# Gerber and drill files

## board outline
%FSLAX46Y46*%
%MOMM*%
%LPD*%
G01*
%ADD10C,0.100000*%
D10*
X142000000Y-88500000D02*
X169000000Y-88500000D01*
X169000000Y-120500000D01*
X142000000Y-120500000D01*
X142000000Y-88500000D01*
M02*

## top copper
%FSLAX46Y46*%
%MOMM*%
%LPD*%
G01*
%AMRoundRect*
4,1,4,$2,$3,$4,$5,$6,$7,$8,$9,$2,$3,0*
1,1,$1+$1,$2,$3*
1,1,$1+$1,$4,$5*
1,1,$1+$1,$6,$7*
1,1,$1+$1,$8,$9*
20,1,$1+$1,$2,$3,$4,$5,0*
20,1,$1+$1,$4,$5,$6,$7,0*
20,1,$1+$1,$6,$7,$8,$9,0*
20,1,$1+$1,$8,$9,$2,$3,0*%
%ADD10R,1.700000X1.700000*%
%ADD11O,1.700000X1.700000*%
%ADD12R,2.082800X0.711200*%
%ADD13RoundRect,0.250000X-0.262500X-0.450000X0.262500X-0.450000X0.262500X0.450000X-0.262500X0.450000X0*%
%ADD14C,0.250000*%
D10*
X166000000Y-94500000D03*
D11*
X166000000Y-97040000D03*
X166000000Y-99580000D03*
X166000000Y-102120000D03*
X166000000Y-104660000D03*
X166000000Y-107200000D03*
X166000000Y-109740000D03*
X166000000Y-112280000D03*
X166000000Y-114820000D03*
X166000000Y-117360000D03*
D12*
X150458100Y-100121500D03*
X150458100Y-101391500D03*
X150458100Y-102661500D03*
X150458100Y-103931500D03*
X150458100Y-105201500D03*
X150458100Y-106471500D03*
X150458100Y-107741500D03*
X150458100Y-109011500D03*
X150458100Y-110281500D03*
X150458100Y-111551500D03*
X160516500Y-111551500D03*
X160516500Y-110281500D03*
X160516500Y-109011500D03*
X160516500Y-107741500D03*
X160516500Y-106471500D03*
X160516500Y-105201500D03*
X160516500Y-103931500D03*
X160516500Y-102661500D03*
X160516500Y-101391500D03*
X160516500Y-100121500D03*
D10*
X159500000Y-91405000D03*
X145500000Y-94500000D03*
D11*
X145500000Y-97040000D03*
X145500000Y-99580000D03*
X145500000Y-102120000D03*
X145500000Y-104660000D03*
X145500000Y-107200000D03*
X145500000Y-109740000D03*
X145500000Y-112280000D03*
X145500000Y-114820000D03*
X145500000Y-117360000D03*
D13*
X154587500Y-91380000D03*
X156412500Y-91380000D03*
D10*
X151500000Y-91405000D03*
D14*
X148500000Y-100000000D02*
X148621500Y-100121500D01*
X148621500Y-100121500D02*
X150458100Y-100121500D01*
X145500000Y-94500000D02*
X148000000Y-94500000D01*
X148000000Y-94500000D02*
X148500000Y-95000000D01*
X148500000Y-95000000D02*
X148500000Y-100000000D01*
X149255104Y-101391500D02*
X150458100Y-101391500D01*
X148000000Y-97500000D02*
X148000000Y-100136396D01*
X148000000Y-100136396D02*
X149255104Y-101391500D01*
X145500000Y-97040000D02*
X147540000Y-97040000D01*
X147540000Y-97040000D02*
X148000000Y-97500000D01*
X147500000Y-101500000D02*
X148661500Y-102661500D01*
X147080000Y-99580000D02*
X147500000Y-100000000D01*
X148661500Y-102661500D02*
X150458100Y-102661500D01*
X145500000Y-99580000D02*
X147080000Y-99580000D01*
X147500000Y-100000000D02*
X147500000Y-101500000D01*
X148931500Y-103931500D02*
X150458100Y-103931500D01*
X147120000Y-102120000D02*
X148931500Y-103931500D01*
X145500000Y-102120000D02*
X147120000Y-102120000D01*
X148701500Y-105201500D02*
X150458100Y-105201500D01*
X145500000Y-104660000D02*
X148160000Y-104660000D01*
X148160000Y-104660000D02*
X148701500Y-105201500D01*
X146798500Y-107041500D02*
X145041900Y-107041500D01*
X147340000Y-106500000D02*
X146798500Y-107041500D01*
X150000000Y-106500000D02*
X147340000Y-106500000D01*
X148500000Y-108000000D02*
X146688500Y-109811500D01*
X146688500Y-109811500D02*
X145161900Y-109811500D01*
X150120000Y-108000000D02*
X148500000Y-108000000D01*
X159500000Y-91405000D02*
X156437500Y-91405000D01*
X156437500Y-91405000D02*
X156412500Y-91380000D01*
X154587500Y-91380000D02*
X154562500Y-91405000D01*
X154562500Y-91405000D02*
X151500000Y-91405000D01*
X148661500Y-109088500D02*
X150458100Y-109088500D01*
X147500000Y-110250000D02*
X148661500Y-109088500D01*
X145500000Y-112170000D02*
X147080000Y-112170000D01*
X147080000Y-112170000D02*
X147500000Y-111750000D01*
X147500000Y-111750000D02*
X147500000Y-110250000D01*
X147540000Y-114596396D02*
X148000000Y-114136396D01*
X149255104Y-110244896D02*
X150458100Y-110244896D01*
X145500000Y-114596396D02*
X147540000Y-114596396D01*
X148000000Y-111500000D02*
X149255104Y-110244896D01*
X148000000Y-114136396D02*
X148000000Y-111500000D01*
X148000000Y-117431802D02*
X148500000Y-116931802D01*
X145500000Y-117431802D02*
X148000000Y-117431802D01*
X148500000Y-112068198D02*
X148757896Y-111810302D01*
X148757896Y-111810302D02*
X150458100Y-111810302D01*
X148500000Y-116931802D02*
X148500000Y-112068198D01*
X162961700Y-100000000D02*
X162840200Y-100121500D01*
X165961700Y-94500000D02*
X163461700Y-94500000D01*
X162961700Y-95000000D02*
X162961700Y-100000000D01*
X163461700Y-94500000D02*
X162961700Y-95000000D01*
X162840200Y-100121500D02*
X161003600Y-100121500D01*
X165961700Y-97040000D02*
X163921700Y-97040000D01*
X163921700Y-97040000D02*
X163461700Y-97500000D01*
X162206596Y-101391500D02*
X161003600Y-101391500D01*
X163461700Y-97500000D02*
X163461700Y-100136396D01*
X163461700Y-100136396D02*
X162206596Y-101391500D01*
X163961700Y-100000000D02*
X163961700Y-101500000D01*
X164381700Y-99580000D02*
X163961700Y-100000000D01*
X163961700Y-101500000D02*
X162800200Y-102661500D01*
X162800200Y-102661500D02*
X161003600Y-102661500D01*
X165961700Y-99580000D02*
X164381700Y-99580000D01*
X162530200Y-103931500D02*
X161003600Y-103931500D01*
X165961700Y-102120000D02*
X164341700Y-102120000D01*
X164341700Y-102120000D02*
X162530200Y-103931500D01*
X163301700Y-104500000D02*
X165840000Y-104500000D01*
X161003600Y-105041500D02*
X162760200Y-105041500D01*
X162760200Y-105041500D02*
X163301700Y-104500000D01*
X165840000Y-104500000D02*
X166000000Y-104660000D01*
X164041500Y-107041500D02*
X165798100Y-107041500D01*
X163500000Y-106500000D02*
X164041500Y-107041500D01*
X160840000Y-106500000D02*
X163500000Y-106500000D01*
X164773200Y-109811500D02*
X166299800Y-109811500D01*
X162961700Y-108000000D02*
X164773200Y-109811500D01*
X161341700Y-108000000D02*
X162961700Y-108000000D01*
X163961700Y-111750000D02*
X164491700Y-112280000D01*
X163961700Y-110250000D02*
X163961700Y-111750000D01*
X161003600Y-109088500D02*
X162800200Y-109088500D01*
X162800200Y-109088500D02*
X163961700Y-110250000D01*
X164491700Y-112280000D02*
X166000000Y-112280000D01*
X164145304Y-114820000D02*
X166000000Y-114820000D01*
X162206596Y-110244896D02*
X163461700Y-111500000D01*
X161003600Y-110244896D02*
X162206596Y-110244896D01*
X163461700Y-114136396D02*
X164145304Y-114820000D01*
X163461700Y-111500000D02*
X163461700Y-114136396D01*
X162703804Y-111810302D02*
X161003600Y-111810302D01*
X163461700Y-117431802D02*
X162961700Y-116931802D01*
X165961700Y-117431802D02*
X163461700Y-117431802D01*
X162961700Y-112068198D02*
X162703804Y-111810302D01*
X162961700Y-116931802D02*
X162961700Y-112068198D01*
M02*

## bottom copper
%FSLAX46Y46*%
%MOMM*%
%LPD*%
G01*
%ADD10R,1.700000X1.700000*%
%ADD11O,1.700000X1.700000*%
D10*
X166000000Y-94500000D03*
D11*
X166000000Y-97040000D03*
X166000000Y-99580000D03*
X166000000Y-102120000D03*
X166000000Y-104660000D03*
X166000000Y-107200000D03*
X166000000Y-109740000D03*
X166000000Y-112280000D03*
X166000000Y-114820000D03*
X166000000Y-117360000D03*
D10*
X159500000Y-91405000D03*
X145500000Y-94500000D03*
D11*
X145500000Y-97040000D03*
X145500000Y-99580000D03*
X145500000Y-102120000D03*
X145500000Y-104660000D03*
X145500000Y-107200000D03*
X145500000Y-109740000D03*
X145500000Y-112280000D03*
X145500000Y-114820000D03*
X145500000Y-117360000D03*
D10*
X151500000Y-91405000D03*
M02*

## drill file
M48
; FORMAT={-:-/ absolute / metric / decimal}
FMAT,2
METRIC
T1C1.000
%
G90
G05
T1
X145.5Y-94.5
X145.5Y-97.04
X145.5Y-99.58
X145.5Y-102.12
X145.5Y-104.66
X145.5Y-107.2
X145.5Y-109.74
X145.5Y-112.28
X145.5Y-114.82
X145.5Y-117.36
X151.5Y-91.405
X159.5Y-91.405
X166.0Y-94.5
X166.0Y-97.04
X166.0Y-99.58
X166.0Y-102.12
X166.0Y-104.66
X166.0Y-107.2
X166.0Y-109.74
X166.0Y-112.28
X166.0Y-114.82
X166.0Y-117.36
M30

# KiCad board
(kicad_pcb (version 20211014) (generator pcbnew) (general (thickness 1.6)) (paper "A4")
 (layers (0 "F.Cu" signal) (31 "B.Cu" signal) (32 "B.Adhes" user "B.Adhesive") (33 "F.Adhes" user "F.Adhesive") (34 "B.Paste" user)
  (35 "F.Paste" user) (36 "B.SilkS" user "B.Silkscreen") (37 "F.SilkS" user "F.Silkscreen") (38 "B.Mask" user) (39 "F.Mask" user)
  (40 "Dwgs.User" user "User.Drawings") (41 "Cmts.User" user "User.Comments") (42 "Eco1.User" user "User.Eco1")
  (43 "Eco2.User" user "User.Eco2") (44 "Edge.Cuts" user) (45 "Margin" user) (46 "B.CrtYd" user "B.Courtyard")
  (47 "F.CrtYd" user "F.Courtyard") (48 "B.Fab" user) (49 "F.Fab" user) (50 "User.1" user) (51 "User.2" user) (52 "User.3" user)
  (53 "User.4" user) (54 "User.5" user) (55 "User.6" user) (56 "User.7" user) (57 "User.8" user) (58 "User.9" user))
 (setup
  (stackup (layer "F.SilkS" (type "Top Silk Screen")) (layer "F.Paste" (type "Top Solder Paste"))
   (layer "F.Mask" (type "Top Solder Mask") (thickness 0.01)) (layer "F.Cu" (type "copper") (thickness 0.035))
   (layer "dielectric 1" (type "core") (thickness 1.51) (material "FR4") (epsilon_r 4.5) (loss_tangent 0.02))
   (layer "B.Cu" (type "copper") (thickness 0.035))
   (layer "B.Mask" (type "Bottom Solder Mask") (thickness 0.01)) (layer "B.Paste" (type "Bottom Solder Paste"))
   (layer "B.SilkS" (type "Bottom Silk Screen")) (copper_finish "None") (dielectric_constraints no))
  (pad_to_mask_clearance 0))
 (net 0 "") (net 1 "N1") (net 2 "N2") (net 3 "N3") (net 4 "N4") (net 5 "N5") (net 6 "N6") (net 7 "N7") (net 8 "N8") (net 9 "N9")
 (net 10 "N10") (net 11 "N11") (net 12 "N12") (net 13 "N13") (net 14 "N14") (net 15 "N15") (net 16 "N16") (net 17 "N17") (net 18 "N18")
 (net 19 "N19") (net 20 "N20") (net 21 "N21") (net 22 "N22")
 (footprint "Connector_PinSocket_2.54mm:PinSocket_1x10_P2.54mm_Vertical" (layer "F.Cu") (at 166 94.5)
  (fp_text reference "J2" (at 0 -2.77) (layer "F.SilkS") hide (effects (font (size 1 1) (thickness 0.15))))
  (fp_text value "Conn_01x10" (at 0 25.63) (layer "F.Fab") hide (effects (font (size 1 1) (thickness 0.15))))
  (pad "1" thru_hole rect (at 0 0) (size 1.7 1.7) (drill 1) (layers *.Cu *.Mask) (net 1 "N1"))
  (pad "2" thru_hole oval (at 0 2.54) (size 1.7 1.7) (drill 1) (layers *.Cu *.Mask) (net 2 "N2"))
  (pad "3" thru_hole oval (at 0 5.08) (size 1.7 1.7) (drill 1) (layers *.Cu *.Mask) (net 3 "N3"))
  (pad "4" thru_hole oval (at 0 7.62) (size 1.7 1.7) (drill 1) (layers *.Cu *.Mask) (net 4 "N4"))
  (pad "5" thru_hole oval (at 0 10.16) (size 1.7 1.7) (drill 1) (layers *.Cu *.Mask) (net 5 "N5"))
  (pad "6" thru_hole oval (at 0 12.7) (size 1.7 1.7) (drill 1) (layers *.Cu *.Mask) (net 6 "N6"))
  (pad "7" thru_hole oval (at 0 15.24) (size 1.7 1.7) (drill 1) (layers *.Cu *.Mask) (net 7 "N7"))
  (pad "8" thru_hole oval (at 0 17.78) (size 1.7 1.7) (drill 1) (layers *.Cu *.Mask) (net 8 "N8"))
  (pad "9" thru_hole oval (at 0 20.32) (size 1.7 1.7) (drill 1) (layers *.Cu *.Mask) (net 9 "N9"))
  (pad "10" thru_hole oval (at 0 22.86) (size 1.7 1.7) (drill 1) (layers *.Cu *.Mask) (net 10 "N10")))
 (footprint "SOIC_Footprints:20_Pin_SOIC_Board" (layer "F.Cu") (at 156.1985 105.8365)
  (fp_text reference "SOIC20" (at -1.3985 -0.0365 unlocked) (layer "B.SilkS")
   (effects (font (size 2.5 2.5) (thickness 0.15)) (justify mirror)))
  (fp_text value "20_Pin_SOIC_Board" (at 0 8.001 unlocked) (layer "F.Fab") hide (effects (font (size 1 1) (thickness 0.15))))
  (pad "1" smd rect (at -5.7404 -5.715) (size 2.0828 0.7112) (layers "F.Cu" "F.Paste" "F.Mask") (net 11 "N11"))
  (pad "2" smd rect (at -5.7404 -4.445) (size 2.0828 0.7112) (layers "F.Cu" "F.Paste" "F.Mask") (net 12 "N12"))
  (pad "3" smd rect (at -5.7404 -3.175) (size 2.0828 0.7112) (layers "F.Cu" "F.Paste" "F.Mask") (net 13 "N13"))
  (pad "4" smd rect (at -5.7404 -1.905) (size 2.0828 0.7112) (layers "F.Cu" "F.Paste" "F.Mask") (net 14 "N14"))
  (pad "5" smd rect (at -5.7404 -0.635) (size 2.0828 0.7112) (layers "F.Cu" "F.Paste" "F.Mask") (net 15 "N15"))
  (pad "6" smd rect (at -5.7404 0.635) (size 2.0828 0.7112) (layers "F.Cu" "F.Paste" "F.Mask") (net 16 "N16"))
  (pad "7" smd rect (at -5.7404 1.905) (size 2.0828 0.7112) (layers "F.Cu" "F.Paste" "F.Mask") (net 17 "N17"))
  (pad "8" smd rect (at -5.7404 3.175) (size 2.0828 0.7112) (layers "F.Cu" "F.Paste" "F.Mask") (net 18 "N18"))
  (pad "9" smd rect (at -5.7404 4.445) (size 2.0828 0.7112) (layers "F.Cu" "F.Paste" "F.Mask") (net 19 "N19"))
  (pad "10" smd rect (at -5.7404 5.715) (size 2.0828 0.7112) (layers "F.Cu" "F.Paste" "F.Mask") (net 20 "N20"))
  (pad "11" smd rect (at 4.318 5.715) (size 2.0828 0.7112) (layers "F.Cu" "F.Paste" "F.Mask") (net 10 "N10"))
  (pad "12" smd rect (at 4.318 4.445) (size 2.0828 0.7112) (layers "F.Cu" "F.Paste" "F.Mask") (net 9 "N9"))
  (pad "13" smd rect (at 4.318 3.175) (size 2.0828 0.7112) (layers "F.Cu" "F.Paste" "F.Mask") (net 8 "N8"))
  (pad "14" smd rect (at 4.318 1.905) (size 2.0828 0.7112) (layers "F.Cu" "F.Paste" "F.Mask") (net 7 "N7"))
  (pad "15" smd rect (at 4.318 0.635) (size 2.0828 0.7112) (layers "F.Cu" "F.Paste" "F.Mask") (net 6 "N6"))
  (pad "16" smd rect (at 4.318 -0.635) (size 2.0828 0.7112) (layers "F.Cu" "F.Paste" "F.Mask") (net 5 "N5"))
  (pad "17" smd rect (at 4.318 -1.905) (size 2.0828 0.7112) (layers "F.Cu" "F.Paste" "F.Mask") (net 4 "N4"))
  (pad "18" smd rect (at 4.318 -3.175) (size 2.0828 0.7112) (layers "F.Cu" "F.Paste" "F.Mask") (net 3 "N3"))
  (pad "19" smd rect (at 4.318 -4.445) (size 2.0828 0.7112) (layers "F.Cu" "F.Paste" "F.Mask") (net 2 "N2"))
  (pad "20" smd rect (at 4.318 -5.715) (size 2.0828 0.7112) (layers "F.Cu" "F.Paste" "F.Mask") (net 1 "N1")))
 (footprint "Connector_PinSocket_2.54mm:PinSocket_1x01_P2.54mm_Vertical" (layer "F.Cu") (at 159.5 91.405)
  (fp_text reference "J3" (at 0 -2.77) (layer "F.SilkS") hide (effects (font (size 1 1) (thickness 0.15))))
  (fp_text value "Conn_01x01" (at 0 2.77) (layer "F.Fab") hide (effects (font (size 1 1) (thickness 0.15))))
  (pad "1" thru_hole rect (at 0 0) (size 1.7 1.7) (drill 1) (layers *.Cu *.Mask) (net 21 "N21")))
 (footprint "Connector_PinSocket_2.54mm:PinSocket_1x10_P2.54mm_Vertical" (layer "F.Cu") (at 145.5 94.5)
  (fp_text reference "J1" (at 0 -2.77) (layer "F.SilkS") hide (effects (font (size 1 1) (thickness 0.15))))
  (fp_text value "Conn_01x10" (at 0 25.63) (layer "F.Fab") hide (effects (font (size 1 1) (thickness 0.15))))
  (pad "1" thru_hole rect (at 0 0) (size 1.7 1.7) (drill 1) (layers *.Cu *.Mask) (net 11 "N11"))
  (pad "2" thru_hole oval (at 0 2.54) (size 1.7 1.7) (drill 1) (layers *.Cu *.Mask) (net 12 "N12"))
  (pad "3" thru_hole oval (at 0 5.08) (size 1.7 1.7) (drill 1) (layers *.Cu *.Mask) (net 13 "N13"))
  (pad "4" thru_hole oval (at 0 7.62) (size 1.7 1.7) (drill 1) (layers *.Cu *.Mask) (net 14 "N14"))
  (pad "5" thru_hole oval (at 0 10.16) (size 1.7 1.7) (drill 1) (layers *.Cu *.Mask) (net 15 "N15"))
  (pad "6" thru_hole oval (at 0 12.7) (size 1.7 1.7) (drill 1) (layers *.Cu *.Mask) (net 16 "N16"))
  (pad "7" thru_hole oval (at 0 15.24) (size 1.7 1.7) (drill 1) (layers *.Cu *.Mask) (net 17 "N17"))
  (pad "8" thru_hole oval (at 0 17.78) (size 1.7 1.7) (drill 1) (layers *.Cu *.Mask) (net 18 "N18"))
  (pad "9" thru_hole oval (at 0 20.32) (size 1.7 1.7) (drill 1) (layers *.Cu *.Mask) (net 19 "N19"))
  (pad "10" thru_hole oval (at 0 22.86) (size 1.7 1.7) (drill 1) (layers *.Cu *.Mask) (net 20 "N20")))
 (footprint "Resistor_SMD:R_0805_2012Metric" (layer "F.Cu") (at 155.5 91.38)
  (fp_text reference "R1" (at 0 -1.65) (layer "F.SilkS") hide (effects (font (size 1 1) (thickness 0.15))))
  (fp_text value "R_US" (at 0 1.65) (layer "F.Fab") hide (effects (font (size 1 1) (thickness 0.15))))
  (pad "1" smd roundrect (at -0.9125 0) (size 1.025 1.4) (layers "F.Cu" "F.Paste" "F.Mask") (roundrect_rratio 0.243902) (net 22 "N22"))
  (pad "2" smd roundrect (at 0.9125 0) (size 1.025 1.4) (layers "F.Cu" "F.Paste" "F.Mask") (roundrect_rratio 0.243902) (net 21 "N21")))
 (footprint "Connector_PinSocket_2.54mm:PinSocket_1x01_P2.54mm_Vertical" (layer "F.Cu") (at 151.5 91.405)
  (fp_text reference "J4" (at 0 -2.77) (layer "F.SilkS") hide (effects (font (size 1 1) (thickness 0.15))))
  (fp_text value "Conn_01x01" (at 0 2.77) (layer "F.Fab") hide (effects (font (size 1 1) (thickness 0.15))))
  (pad "1" thru_hole rect (at 0 0) (size 1.7 1.7) (drill 1) (layers *.Cu *.Mask) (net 22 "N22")))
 (gr_rect (start 142 88.5) (end 169 120.5) (layer "Edge.Cuts") (width 0.1) (fill none))
 (segment (start 148.5 100) (end 148.6215 100.1215) (width 0.25) (layer "F.Cu") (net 11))
 (segment (start 148.6215 100.1215) (end 150.4581 100.1215) (width 0.25) (layer "F.Cu") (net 11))
 (segment (start 145.5 94.5) (end 148 94.5) (width 0.25) (layer "F.Cu") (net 11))
 (segment (start 148 94.5) (end 148.5 95) (width 0.25) (layer "F.Cu") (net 11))
 (segment (start 148.5 95) (end 148.5 100) (width 0.25) (layer "F.Cu") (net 11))
 (segment (start 149.255104 101.3915) (end 150.4581 101.3915) (width 0.25) (layer "F.Cu") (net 12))
 (segment (start 148 97.5) (end 148 100.136396) (width 0.25) (layer "F.Cu") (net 12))
 (segment (start 148 100.136396) (end 149.255104 101.3915) (width 0.25) (layer "F.Cu") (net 12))
 (segment (start 145.5 97.04) (end 147.54 97.04) (width 0.25) (layer "F.Cu") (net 12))
 (segment (start 147.54 97.04) (end 148 97.5) (width 0.25) (layer "F.Cu") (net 12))
 (segment (start 147.5 101.5) (end 148.6615 102.6615) (width 0.25) (layer "F.Cu") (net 13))
 (segment (start 147.08 99.58) (end 147.5 100) (width 0.25) (layer "F.Cu") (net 13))
 (segment (start 148.6615 102.6615) (end 150.4581 102.6615) (width 0.25) (layer "F.Cu") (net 13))
 (segment (start 145.5 99.58) (end 147.08 99.58) (width 0.25) (layer "F.Cu") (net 13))
 (segment (start 147.5 100) (end 147.5 101.5) (width 0.25) (layer "F.Cu") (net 13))
 (segment (start 148.9315 103.9315) (end 150.4581 103.9315) (width 0.25) (layer "F.Cu") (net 14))
 (segment (start 147.12 102.12) (end 148.9315 103.9315) (width 0.25) (layer "F.Cu") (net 14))
 (segment (start 145.5 102.12) (end 147.12 102.12) (width 0.25) (layer "F.Cu") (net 14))
 (segment (start 148.7015 105.2015) (end 150.4581 105.2015) (width 0.25) (layer "F.Cu") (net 15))
 (segment (start 145.5 104.66) (end 148.16 104.66) (width 0.25) (layer "F.Cu") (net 15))
 (segment (start 148.16 104.66) (end 148.7015 105.2015) (width 0.25) (layer "F.Cu") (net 15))
 (segment (start 146.7985 107.0415) (end 145.0419 107.0415) (width 0.25) (layer "F.Cu") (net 16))
 (segment (start 147.34 106.5) (end 146.7985 107.0415) (width 0.25) (layer "F.Cu") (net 16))
 (segment (start 150 106.5) (end 147.34 106.5) (width 0.25) (layer "F.Cu") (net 16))
 (segment (start 148.5 108) (end 146.6885 109.8115) (width 0.25) (layer "F.Cu") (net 17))
 (segment (start 146.6885 109.8115) (end 145.1619 109.8115) (width 0.25) (layer "F.Cu") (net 17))
 (segment (start 150.12 108) (end 148.5 108) (width 0.25) (layer "F.Cu") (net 17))
 (segment (start 159.5 91.405) (end 156.4375 91.405) (width 0.25) (layer "F.Cu") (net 21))
 (segment (start 156.4375 91.405) (end 156.4125 91.38) (width 0.25) (layer "F.Cu") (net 21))
 (segment (start 154.5875 91.38) (end 154.5625 91.405) (width 0.25) (layer "F.Cu") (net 22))
 (segment (start 154.5625 91.405) (end 151.5 91.405) (width 0.25) (layer "F.Cu") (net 22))
 (segment (start 148.6615 109.0885) (end 150.4581 109.0885) (width 0.25) (layer "F.Cu") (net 18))
 (segment (start 147.5 110.25) (end 148.6615 109.0885) (width 0.25) (layer "F.Cu") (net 18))
 (segment (start 145.5 112.17) (end 147.08 112.17) (width 0.25) (layer "F.Cu") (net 18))
 (segment (start 147.08 112.17) (end 147.5 111.75) (width 0.25) (layer "F.Cu") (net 18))
 (segment (start 147.5 111.75) (end 147.5 110.25) (width 0.25) (layer "F.Cu") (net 18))
 (segment (start 147.54 114.596396) (end 148 114.136396) (width 0.25) (layer "F.Cu") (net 19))
 (segment (start 149.255104 110.244896) (end 150.4581 110.244896) (width 0.25) (layer "F.Cu") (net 19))
 (segment (start 145.5 114.596396) (end 147.54 114.596396) (width 0.25) (layer "F.Cu") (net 19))
 (segment (start 148 111.5) (end 149.255104 110.244896) (width 0.25) (layer "F.Cu") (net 19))
 (segment (start 148 114.136396) (end 148 111.5) (width 0.25) (layer "F.Cu") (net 19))
 (segment (start 148 117.431802) (end 148.5 116.931802) (width 0.25) (layer "F.Cu") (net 20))
 (segment (start 145.5 117.431802) (end 148 117.431802) (width 0.25) (layer "F.Cu") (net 20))
 (segment (start 148.5 112.068198) (end 148.757896 111.810302) (width 0.25) (layer "F.Cu") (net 20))
 (segment (start 148.757896 111.810302) (end 150.4581 111.810302) (width 0.25) (layer "F.Cu") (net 20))
 (segment (start 148.5 116.931802) (end 148.5 112.068198) (width 0.25) (layer "F.Cu") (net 20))
 (segment (start 162.9617 100) (end 162.8402 100.1215) (width 0.25) (layer "F.Cu") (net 1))
 (segment (start 165.9617 94.5) (end 163.4617 94.5) (width 0.25) (layer "F.Cu") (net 1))
 (segment (start 162.9617 95) (end 162.9617 100) (width 0.25) (layer "F.Cu") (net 1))
 (segment (start 163.4617 94.5) (end 162.9617 95) (width 0.25) (layer "F.Cu") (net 1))
 (segment (start 162.8402 100.1215) (end 161.0036 100.1215) (width 0.25) (layer "F.Cu") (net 1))
 (segment (start 165.9617 97.04) (end 163.9217 97.04) (width 0.25) (layer "F.Cu") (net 2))
 (segment (start 163.9217 97.04) (end 163.4617 97.5) (width 0.25) (layer "F.Cu") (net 2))
 (segment (start 162.206596 101.3915) (end 161.0036 101.3915) (width 0.25) (layer "F.Cu") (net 2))
 (segment (start 163.4617 97.5) (end 163.4617 100.136396) (width 0.25) (layer "F.Cu") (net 2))
 (segment (start 163.4617 100.136396) (end 162.206596 101.3915) (width 0.25) (layer "F.Cu") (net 2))
 (segment (start 163.9617 100) (end 163.9617 101.5) (width 0.25) (layer "F.Cu") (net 3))
 (segment (start 164.3817 99.58) (end 163.9617 100) (width 0.25) (layer "F.Cu") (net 3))
 (segment (start 163.9617 101.5) (end 162.8002 102.6615) (width 0.25) (layer "F.Cu") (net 3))
 (segment (start 162.8002 102.6615) (end 161.0036 102.6615) (width 0.25) (layer "F.Cu") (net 3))
 (segment (start 165.9617 99.58) (end 164.3817 99.58) (width 0.25) (layer "F.Cu") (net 3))
 (segment (start 162.5302 103.9315) (end 161.0036 103.9315) (width 0.25) (layer "F.Cu") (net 4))
 (segment (start 165.9617 102.12) (end 164.3417 102.12) (width 0.25) (layer "F.Cu") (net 4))
 (segment (start 164.3417 102.12) (end 162.5302 103.9315) (width 0.25) (layer "F.Cu") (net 4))
 (segment (start 163.3017 104.5) (end 165.84 104.5) (width 0.25) (layer "F.Cu") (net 5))
 (segment (start 161.0036 105.0415) (end 162.7602 105.0415) (width 0.25) (layer "F.Cu") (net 5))
 (segment (start 162.7602 105.0415) (end 163.3017 104.5) (width 0.25) (layer "F.Cu") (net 5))
 (segment (start 165.84 104.5) (end 166 104.66) (width 0.25) (layer "F.Cu") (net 5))
 (segment (start 164.0415 107.0415) (end 165.7981 107.0415) (width 0.25) (layer "F.Cu") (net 6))
 (segment (start 163.5 106.5) (end 164.0415 107.0415) (width 0.25) (layer "F.Cu") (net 6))
 (segment (start 160.84 106.5) (end 163.5 106.5) (width 0.25) (layer "F.Cu") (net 6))
 (segment (start 164.7732 109.8115) (end 166.2998 109.8115) (width 0.25) (layer "F.Cu") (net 7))
 (segment (start 162.9617 108) (end 164.7732 109.8115) (width 0.25) (layer "F.Cu") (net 7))
 (segment (start 161.3417 108) (end 162.9617 108) (width 0.25) (layer "F.Cu") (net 7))
 (segment (start 163.9617 111.75) (end 164.4917 112.28) (width 0.25) (layer "F.Cu") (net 8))
 (segment (start 163.9617 110.25) (end 163.9617 111.75) (width 0.25) (layer "F.Cu") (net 8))
 (segment (start 161.0036 109.0885) (end 162.8002 109.0885) (width 0.25) (layer "F.Cu") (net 8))
 (segment (start 162.8002 109.0885) (end 163.9617 110.25) (width 0.25) (layer "F.Cu") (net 8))
 (segment (start 164.4917 112.28) (end 166 112.28) (width 0.25) (layer "F.Cu") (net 8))
 (segment (start 164.145304 114.82) (end 166 114.82) (width 0.25) (layer "F.Cu") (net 9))
 (segment (start 162.206596 110.244896) (end 163.4617 111.5) (width 0.25) (layer "F.Cu") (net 9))
 (segment (start 161.0036 110.244896) (end 162.206596 110.244896) (width 0.25) (layer "F.Cu") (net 9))
 (segment (start 163.4617 114.136396) (end 164.145304 114.82) (width 0.25) (layer "F.Cu") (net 9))
 (segment (start 163.4617 111.5) (end 163.4617 114.136396) (width 0.25) (layer "F.Cu") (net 9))
 (segment (start 162.703804 111.810302) (end 161.0036 111.810302) (width 0.25) (layer "F.Cu") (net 10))
 (segment (start 163.4617 117.431802) (end 162.9617 116.931802) (width 0.25) (layer "F.Cu") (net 10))
 (segment (start 165.9617 117.431802) (end 163.4617 117.431802) (width 0.25) (layer "F.Cu") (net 10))
 (segment (start 162.9617 112.068198) (end 162.703804 111.810302) (width 0.25) (layer "F.Cu") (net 10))
 (segment (start 162.9617 116.931802) (end 162.9617 112.068198) (width 0.25) (layer "F.Cu") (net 10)))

